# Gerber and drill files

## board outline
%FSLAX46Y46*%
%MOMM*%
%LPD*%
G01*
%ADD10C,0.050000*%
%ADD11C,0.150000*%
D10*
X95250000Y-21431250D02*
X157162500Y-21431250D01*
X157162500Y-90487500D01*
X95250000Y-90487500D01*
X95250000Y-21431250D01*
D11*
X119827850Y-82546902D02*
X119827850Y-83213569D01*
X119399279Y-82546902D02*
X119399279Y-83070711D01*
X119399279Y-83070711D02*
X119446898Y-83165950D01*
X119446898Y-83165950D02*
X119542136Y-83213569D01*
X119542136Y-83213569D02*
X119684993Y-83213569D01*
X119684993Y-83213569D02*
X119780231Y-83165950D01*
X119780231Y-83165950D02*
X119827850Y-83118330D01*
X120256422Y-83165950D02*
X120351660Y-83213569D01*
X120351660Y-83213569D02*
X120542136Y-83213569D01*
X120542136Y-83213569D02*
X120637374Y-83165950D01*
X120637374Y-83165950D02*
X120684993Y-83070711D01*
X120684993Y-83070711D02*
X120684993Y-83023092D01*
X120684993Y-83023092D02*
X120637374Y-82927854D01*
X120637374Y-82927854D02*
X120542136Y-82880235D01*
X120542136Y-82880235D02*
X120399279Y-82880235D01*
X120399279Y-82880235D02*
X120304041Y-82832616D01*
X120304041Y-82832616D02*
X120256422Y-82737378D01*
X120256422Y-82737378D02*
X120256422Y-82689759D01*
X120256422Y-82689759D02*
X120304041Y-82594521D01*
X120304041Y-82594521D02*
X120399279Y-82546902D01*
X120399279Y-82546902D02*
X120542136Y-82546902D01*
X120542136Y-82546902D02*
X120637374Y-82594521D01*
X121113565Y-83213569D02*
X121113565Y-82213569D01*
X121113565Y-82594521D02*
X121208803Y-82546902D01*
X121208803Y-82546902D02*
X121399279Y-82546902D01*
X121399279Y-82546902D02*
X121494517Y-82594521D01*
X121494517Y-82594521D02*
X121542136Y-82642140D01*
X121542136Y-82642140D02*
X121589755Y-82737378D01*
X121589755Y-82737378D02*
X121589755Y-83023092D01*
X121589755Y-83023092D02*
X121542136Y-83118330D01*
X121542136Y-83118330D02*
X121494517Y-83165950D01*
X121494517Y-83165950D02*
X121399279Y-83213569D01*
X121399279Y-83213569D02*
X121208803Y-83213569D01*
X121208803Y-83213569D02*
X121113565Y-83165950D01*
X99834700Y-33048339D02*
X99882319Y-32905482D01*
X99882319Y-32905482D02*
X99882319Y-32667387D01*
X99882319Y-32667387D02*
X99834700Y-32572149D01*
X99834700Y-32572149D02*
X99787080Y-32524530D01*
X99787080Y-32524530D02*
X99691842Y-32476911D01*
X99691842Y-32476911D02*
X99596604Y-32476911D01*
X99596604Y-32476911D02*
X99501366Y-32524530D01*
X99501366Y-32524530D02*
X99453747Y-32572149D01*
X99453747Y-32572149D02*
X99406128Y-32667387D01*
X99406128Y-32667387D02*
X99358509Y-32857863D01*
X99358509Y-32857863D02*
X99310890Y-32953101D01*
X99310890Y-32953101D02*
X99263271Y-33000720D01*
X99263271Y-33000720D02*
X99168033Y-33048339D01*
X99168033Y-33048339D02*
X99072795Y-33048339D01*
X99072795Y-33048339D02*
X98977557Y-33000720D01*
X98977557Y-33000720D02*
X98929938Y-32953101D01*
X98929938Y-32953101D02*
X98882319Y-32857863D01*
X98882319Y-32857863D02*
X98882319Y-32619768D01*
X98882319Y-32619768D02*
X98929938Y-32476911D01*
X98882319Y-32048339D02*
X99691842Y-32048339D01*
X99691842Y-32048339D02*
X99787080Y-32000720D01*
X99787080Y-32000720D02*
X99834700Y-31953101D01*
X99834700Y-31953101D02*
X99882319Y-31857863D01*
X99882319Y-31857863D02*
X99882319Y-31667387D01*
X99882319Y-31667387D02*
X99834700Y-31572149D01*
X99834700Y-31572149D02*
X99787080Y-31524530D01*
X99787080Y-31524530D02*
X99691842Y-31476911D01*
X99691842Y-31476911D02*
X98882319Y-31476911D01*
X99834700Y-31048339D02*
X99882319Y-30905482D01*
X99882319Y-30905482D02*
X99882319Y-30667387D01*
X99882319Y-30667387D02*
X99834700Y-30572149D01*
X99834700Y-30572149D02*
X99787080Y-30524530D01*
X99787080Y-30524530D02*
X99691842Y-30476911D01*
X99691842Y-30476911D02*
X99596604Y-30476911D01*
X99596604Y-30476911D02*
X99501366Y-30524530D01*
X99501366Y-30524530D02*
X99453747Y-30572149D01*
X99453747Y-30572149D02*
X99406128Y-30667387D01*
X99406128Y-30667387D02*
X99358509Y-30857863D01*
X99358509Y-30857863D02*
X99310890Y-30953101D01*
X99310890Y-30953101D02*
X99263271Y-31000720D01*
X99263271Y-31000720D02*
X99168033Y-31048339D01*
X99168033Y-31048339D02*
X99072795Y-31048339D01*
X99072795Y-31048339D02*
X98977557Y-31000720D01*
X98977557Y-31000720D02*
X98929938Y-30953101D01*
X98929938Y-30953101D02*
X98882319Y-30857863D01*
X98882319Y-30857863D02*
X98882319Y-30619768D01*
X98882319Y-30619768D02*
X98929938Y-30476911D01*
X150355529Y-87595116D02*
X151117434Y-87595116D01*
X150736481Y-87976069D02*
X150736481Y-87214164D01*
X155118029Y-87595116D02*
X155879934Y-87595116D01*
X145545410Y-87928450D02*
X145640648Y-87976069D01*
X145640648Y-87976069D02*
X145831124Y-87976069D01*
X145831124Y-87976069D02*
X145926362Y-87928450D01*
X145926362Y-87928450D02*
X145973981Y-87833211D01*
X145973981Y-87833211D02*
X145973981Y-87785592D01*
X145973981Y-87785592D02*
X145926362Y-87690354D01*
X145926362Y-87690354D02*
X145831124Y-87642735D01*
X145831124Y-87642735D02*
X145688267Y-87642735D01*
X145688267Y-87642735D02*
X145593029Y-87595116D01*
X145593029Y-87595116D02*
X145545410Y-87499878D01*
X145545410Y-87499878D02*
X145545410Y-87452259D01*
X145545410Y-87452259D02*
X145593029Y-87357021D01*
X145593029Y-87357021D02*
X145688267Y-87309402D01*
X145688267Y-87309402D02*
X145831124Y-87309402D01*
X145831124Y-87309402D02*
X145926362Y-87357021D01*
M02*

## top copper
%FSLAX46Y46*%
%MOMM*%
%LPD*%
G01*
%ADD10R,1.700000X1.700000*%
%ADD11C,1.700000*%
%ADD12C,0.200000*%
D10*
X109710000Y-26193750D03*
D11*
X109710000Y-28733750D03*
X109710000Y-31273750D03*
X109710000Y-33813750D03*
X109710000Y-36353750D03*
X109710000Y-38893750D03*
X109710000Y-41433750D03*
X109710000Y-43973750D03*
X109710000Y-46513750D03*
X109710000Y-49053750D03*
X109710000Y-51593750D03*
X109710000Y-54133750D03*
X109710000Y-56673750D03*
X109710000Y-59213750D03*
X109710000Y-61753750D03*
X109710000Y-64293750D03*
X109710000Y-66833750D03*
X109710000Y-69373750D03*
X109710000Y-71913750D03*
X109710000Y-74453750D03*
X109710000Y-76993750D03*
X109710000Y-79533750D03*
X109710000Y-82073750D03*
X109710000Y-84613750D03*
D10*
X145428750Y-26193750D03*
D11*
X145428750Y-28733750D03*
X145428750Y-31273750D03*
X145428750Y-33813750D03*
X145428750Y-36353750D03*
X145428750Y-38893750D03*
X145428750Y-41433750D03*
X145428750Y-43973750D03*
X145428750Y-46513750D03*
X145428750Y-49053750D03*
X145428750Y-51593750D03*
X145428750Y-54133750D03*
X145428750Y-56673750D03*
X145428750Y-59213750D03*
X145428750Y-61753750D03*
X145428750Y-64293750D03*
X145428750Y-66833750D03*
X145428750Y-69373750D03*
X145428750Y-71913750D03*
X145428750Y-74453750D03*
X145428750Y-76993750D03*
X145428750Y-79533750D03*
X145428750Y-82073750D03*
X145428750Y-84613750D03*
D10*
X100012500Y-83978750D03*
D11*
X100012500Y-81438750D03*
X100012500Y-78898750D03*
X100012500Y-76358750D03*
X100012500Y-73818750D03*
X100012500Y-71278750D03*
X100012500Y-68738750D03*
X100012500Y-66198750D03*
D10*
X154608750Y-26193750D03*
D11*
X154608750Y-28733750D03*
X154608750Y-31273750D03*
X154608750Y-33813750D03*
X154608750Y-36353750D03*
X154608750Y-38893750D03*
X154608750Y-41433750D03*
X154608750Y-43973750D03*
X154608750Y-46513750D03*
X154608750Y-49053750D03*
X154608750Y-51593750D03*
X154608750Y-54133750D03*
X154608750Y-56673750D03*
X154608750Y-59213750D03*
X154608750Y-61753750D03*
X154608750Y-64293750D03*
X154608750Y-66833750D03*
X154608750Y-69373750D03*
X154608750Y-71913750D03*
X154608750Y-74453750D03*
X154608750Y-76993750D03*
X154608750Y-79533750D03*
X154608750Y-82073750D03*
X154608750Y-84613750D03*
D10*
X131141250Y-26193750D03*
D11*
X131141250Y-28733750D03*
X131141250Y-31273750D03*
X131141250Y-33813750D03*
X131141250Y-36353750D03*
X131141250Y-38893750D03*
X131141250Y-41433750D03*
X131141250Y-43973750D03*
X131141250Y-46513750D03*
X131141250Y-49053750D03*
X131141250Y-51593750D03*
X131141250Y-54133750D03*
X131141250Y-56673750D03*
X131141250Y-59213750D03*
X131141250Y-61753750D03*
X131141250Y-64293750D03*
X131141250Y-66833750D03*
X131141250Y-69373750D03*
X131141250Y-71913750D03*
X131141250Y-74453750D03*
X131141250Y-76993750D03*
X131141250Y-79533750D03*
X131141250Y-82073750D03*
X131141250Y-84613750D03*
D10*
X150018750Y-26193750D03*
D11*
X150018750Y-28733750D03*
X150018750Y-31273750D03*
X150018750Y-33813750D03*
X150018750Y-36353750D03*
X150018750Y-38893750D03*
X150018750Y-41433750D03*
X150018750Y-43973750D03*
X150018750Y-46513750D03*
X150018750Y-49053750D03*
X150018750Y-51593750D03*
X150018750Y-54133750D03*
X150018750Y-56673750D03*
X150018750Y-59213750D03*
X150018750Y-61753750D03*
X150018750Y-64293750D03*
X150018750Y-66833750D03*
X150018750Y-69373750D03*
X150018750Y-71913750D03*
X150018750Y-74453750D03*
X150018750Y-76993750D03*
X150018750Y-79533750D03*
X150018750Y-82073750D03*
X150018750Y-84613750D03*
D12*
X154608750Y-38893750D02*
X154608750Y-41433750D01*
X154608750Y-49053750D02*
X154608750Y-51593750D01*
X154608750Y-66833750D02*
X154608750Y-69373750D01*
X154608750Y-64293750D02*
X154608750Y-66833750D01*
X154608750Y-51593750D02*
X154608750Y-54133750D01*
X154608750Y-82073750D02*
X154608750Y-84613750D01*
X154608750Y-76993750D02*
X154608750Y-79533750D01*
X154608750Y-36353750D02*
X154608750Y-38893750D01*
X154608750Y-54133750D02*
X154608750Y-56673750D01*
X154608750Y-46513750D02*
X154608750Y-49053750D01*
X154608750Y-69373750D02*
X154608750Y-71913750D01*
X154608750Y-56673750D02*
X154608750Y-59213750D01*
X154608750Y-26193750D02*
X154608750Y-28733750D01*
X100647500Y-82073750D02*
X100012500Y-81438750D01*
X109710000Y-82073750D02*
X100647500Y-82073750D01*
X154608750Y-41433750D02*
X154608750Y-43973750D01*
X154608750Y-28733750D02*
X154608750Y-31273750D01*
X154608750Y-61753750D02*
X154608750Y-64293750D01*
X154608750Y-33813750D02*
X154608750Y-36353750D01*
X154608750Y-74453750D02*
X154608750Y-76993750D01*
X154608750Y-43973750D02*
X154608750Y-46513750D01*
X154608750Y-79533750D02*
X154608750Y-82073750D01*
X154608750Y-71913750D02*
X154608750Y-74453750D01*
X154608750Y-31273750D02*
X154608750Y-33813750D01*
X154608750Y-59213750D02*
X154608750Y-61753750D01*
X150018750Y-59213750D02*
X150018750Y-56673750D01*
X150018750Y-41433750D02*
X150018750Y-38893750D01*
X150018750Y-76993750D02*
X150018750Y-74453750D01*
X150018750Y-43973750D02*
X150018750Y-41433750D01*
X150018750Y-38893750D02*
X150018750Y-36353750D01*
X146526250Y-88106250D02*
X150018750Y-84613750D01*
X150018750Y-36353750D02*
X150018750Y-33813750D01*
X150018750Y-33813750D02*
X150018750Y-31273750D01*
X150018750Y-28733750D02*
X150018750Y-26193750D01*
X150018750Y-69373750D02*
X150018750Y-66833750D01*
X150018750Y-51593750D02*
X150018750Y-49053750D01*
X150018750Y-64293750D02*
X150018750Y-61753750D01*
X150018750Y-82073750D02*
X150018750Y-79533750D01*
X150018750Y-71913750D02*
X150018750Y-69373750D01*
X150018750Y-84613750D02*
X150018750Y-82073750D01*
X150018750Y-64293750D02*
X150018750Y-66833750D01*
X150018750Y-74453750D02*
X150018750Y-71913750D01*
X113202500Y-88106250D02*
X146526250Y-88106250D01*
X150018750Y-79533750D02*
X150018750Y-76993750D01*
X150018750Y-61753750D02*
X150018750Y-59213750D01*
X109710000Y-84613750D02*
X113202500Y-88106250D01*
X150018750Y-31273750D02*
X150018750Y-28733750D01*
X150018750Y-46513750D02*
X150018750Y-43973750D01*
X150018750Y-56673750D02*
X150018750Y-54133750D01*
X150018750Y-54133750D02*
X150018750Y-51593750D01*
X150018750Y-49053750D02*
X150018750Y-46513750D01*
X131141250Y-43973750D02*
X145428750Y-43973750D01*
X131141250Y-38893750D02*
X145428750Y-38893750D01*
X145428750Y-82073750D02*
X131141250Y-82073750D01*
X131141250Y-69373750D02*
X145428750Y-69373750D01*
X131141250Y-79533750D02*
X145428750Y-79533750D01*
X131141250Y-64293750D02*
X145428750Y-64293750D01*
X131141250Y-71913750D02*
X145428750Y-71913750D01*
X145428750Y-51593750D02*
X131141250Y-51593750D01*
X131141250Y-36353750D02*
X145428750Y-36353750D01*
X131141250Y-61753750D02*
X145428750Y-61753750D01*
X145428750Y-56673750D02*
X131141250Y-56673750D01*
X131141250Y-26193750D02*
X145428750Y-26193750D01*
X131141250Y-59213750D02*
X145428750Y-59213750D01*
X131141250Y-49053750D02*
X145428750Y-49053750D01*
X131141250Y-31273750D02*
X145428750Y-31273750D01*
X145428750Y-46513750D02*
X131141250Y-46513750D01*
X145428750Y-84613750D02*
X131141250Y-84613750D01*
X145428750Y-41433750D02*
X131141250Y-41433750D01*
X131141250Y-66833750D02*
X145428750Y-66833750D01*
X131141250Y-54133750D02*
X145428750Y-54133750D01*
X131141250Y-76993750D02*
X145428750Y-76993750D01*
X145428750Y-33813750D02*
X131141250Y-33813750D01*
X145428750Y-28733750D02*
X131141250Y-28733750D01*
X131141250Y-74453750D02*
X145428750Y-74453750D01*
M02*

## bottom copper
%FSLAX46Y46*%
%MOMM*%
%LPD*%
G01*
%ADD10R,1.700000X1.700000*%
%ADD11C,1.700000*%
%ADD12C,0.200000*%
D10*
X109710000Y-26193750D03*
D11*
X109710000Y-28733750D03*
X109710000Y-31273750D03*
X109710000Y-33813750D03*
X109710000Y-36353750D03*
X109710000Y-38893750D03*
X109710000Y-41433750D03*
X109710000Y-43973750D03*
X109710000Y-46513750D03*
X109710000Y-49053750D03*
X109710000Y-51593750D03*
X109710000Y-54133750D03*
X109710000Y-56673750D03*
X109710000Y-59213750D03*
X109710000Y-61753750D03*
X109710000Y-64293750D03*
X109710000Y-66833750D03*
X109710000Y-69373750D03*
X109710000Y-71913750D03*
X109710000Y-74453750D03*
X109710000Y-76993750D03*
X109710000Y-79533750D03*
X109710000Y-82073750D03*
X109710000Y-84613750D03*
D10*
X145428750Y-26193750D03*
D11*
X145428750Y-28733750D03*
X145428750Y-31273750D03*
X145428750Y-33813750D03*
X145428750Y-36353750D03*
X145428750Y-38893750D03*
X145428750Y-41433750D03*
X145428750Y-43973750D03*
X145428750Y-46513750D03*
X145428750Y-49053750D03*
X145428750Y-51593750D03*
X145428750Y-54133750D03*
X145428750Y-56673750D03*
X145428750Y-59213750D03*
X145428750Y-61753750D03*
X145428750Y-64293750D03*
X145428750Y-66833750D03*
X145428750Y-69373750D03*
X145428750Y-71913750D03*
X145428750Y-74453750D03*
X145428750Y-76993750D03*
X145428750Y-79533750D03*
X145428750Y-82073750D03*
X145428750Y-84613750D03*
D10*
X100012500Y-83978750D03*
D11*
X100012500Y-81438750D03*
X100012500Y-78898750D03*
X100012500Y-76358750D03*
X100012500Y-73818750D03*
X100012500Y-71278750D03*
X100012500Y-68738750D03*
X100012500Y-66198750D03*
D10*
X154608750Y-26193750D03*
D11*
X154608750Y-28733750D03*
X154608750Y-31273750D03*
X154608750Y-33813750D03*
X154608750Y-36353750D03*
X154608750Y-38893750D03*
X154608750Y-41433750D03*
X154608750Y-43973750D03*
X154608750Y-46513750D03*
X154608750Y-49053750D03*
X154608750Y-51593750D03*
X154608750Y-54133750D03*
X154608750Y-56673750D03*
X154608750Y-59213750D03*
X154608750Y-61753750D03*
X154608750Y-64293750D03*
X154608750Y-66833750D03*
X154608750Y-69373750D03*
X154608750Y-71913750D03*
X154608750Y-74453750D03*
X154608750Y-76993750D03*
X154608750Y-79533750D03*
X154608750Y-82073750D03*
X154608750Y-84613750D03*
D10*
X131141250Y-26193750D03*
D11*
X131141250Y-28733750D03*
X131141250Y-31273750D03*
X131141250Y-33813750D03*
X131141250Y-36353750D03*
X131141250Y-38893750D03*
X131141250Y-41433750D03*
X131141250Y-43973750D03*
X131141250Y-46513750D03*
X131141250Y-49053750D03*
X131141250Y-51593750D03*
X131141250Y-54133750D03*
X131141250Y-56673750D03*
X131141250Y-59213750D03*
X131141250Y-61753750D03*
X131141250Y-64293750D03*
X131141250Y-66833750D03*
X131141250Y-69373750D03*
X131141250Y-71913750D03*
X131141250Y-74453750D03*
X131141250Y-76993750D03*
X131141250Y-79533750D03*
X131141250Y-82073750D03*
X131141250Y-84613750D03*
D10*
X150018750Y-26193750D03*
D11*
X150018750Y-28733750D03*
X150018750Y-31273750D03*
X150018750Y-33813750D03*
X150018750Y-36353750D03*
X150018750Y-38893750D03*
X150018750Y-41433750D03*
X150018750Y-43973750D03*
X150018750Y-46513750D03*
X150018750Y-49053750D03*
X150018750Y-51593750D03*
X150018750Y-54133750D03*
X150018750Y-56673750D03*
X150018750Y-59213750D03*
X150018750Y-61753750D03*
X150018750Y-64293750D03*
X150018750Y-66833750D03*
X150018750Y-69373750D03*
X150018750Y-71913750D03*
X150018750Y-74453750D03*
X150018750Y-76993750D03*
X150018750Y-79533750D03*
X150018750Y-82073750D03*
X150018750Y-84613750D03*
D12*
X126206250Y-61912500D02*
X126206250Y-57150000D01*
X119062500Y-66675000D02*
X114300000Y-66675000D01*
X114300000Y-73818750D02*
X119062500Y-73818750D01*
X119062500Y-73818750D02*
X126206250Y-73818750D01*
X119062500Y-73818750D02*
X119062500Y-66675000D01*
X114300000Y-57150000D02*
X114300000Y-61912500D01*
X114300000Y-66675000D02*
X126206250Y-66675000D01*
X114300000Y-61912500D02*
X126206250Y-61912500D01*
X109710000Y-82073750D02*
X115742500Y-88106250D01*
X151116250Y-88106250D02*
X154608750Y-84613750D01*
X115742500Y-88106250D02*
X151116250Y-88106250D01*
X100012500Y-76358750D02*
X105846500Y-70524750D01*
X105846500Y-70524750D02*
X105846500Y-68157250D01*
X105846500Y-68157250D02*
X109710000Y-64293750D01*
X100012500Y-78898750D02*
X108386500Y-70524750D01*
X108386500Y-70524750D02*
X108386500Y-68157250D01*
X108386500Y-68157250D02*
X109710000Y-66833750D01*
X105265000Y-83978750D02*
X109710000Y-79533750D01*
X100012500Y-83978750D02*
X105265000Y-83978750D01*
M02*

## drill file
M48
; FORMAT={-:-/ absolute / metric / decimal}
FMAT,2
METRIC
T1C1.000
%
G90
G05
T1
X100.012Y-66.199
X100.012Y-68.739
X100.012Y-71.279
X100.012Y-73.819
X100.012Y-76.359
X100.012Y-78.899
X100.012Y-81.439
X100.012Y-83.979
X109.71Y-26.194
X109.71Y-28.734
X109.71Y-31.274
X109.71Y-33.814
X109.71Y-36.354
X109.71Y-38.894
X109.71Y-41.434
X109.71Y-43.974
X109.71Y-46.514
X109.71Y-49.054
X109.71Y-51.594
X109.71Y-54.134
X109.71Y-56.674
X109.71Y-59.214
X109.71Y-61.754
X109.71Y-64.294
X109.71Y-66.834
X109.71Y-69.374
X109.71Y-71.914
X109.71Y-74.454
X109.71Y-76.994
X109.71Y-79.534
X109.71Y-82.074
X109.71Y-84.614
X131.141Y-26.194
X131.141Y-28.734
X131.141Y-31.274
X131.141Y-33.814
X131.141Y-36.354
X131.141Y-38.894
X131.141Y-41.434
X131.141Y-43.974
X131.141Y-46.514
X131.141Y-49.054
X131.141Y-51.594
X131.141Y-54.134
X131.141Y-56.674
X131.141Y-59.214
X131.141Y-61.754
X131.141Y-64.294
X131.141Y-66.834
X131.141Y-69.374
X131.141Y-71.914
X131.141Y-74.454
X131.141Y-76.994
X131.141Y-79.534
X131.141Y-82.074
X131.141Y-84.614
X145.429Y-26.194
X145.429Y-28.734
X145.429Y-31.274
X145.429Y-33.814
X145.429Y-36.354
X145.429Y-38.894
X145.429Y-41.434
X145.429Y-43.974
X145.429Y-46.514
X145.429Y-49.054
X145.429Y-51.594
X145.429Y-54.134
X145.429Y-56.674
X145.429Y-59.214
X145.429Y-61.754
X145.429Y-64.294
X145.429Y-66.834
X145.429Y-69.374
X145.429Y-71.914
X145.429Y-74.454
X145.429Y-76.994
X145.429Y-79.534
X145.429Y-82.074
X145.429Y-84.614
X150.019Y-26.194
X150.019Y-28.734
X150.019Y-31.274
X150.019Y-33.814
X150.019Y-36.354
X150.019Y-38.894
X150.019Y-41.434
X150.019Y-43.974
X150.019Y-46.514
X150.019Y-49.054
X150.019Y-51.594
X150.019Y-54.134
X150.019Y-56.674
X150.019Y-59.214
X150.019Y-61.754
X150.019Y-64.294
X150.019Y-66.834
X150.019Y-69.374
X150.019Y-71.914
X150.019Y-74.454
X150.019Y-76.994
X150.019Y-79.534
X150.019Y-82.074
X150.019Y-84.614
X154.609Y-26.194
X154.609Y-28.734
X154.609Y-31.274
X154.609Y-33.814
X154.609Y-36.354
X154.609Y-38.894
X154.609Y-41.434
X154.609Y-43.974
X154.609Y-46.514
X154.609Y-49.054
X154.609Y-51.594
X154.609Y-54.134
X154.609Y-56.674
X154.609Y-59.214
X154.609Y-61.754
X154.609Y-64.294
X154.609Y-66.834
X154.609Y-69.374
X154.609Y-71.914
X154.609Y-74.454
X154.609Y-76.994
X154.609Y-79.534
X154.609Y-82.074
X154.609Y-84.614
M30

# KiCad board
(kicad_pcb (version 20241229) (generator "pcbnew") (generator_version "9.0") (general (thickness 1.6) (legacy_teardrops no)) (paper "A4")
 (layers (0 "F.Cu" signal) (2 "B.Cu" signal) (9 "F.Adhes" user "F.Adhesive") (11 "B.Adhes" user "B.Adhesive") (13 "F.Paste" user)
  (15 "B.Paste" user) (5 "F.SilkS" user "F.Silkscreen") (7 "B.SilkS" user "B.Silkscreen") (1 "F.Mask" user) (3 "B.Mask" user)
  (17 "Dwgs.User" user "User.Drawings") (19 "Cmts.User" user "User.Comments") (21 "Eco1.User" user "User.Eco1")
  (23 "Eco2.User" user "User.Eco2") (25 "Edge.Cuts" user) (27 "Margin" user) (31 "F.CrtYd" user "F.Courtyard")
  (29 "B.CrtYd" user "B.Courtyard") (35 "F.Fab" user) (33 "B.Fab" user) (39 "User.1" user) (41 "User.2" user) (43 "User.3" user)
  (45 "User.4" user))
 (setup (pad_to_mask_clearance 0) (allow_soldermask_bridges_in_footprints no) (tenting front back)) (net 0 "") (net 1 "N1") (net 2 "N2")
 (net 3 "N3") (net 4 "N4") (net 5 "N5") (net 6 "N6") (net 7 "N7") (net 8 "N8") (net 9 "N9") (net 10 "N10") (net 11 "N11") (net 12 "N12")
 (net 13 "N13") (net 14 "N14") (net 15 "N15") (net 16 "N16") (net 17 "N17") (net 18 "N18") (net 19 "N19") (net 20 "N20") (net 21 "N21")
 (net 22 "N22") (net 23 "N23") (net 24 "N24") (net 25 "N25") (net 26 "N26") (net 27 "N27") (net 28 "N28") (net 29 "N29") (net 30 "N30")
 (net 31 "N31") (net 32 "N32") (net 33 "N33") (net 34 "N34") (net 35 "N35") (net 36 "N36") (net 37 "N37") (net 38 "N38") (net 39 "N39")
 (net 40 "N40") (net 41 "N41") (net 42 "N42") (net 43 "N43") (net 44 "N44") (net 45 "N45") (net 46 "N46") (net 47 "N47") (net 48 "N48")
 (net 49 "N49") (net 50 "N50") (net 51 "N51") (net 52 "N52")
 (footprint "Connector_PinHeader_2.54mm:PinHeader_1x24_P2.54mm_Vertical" (layer "F.Cu") (at 109.71 26.19375)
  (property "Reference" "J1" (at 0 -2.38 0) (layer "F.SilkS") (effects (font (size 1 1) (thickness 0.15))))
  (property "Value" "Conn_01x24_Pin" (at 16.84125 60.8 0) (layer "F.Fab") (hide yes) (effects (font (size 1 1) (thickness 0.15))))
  (pad "1" thru_hole rect (at 0 0) (size 1.7 1.7) (drill 1) (layers "*.Cu" "*.Mask") (remove_unused_layers no) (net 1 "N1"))
  (pad "2" thru_hole circle (at 0 2.54) (size 1.7 1.7) (drill 1) (layers "*.Cu" "*.Mask") (remove_unused_layers no) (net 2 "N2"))
  (pad "3" thru_hole circle (at 0 5.08) (size 1.7 1.7) (drill 1) (layers "*.Cu" "*.Mask") (remove_unused_layers no) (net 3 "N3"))
  (pad "4" thru_hole circle (at 0 7.62) (size 1.7 1.7) (drill 1) (layers "*.Cu" "*.Mask") (remove_unused_layers no) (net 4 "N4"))
  (pad "5" thru_hole circle (at 0 10.16) (size 1.7 1.7) (drill 1) (layers "*.Cu" "*.Mask") (remove_unused_layers no) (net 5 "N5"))
  (pad "6" thru_hole circle (at 0 12.7) (size 1.7 1.7) (drill 1) (layers "*.Cu" "*.Mask") (remove_unused_layers no) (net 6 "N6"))
  (pad "7" thru_hole circle (at 0 15.24) (size 1.7 1.7) (drill 1) (layers "*.Cu" "*.Mask") (remove_unused_layers no) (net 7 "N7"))
  (pad "8" thru_hole circle (at 0 17.78) (size 1.7 1.7) (drill 1) (layers "*.Cu" "*.Mask") (remove_unused_layers no) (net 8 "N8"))
  (pad "9" thru_hole circle (at 0 20.32) (size 1.7 1.7) (drill 1) (layers "*.Cu" "*.Mask") (remove_unused_layers no) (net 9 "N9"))
  (pad "10" thru_hole circle (at 0 22.86) (size 1.7 1.7) (drill 1) (layers "*.Cu" "*.Mask") (remove_unused_layers no) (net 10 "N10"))
  (pad "11" thru_hole circle (at 0 25.4) (size 1.7 1.7) (drill 1) (layers "*.Cu" "*.Mask") (remove_unused_layers no) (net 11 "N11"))
  (pad "12" thru_hole circle (at 0 27.94) (size 1.7 1.7) (drill 1) (layers "*.Cu" "*.Mask") (remove_unused_layers no) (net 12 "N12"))
  (pad "13" thru_hole circle (at 0 30.48) (size 1.7 1.7) (drill 1) (layers "*.Cu" "*.Mask") (remove_unused_layers no) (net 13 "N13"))
  (pad "14" thru_hole circle (at 0 33.02) (size 1.7 1.7) (drill 1) (layers "*.Cu" "*.Mask") (remove_unused_layers no) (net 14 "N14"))
  (pad "15" thru_hole circle (at 0 35.56) (size 1.7 1.7) (drill 1) (layers "*.Cu" "*.Mask") (remove_unused_layers no) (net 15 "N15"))
  (pad "16" thru_hole circle (at 0 38.1) (size 1.7 1.7) (drill 1) (layers "*.Cu" "*.Mask") (remove_unused_layers no) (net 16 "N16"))
  (pad "17" thru_hole circle (at 0 40.64) (size 1.7 1.7) (drill 1) (layers "*.Cu" "*.Mask") (remove_unused_layers no) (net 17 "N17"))
  (pad "18" thru_hole circle (at 0 43.18) (size 1.7 1.7) (drill 1) (layers "*.Cu" "*.Mask") (remove_unused_layers no) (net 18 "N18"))
  (pad "19" thru_hole circle (at 0 45.72) (size 1.7 1.7) (drill 1) (layers "*.Cu" "*.Mask") (remove_unused_layers no) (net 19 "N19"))
  (pad "20" thru_hole circle (at 0 48.26) (size 1.7 1.7) (drill 1) (layers "*.Cu" "*.Mask") (remove_unused_layers no) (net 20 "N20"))
  (pad "21" thru_hole circle (at 0 50.8) (size 1.7 1.7) (drill 1) (layers "*.Cu" "*.Mask") (remove_unused_layers no) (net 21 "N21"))
  (pad "22" thru_hole circle (at 0 53.34) (size 1.7 1.7) (drill 1) (layers "*.Cu" "*.Mask") (remove_unused_layers no) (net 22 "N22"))
  (pad "23" thru_hole circle (at 0 55.88) (size 1.7 1.7) (drill 1) (layers "*.Cu" "*.Mask") (remove_unused_layers no) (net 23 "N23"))
  (pad "24" thru_hole circle (at 0 58.42) (size 1.7 1.7) (drill 1) (layers "*.Cu" "*.Mask") (remove_unused_layers no) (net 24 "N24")))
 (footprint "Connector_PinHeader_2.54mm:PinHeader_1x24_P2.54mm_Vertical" (layer "F.Cu") (at 145.42875 26.19375)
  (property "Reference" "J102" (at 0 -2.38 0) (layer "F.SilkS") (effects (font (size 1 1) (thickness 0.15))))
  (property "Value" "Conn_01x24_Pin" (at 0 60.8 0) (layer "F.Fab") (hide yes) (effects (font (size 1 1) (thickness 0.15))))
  (pad "1" thru_hole rect (at 0 0) (size 1.7 1.7) (drill 1) (layers "*.Cu" "*.Mask") (remove_unused_layers no) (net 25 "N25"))
  (pad "2" thru_hole circle (at 0 2.54) (size 1.7 1.7) (drill 1) (layers "*.Cu" "*.Mask") (remove_unused_layers no) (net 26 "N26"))
  (pad "3" thru_hole circle (at 0 5.08) (size 1.7 1.7) (drill 1) (layers "*.Cu" "*.Mask") (remove_unused_layers no) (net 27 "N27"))
  (pad "4" thru_hole circle (at 0 7.62) (size 1.7 1.7) (drill 1) (layers "*.Cu" "*.Mask") (remove_unused_layers no) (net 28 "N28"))
  (pad "5" thru_hole circle (at 0 10.16) (size 1.7 1.7) (drill 1) (layers "*.Cu" "*.Mask") (remove_unused_layers no) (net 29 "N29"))
  (pad "6" thru_hole circle (at 0 12.7) (size 1.7 1.7) (drill 1) (layers "*.Cu" "*.Mask") (remove_unused_layers no) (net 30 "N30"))
  (pad "7" thru_hole circle (at 0 15.24) (size 1.7 1.7) (drill 1) (layers "*.Cu" "*.Mask") (remove_unused_layers no) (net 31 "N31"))
  (pad "8" thru_hole circle (at 0 17.78) (size 1.7 1.7) (drill 1) (layers "*.Cu" "*.Mask") (remove_unused_layers no) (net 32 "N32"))
  (pad "9" thru_hole circle (at 0 20.32) (size 1.7 1.7) (drill 1) (layers "*.Cu" "*.Mask") (remove_unused_layers no) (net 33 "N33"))
  (pad "10" thru_hole circle (at 0 22.86) (size 1.7 1.7) (drill 1) (layers "*.Cu" "*.Mask") (remove_unused_layers no) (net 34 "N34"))
  (pad "11" thru_hole circle (at 0 25.4) (size 1.7 1.7) (drill 1) (layers "*.Cu" "*.Mask") (remove_unused_layers no) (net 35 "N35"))
  (pad "12" thru_hole circle (at 0 27.94) (size 1.7 1.7) (drill 1) (layers "*.Cu" "*.Mask") (remove_unused_layers no) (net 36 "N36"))
  (pad "13" thru_hole circle (at 0 30.48) (size 1.7 1.7) (drill 1) (layers "*.Cu" "*.Mask") (remove_unused_layers no) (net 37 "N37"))
  (pad "14" thru_hole circle (at 0 33.02) (size 1.7 1.7) (drill 1) (layers "*.Cu" "*.Mask") (remove_unused_layers no) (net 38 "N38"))
  (pad "15" thru_hole circle (at 0 35.56) (size 1.7 1.7) (drill 1) (layers "*.Cu" "*.Mask") (remove_unused_layers no) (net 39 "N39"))
  (pad "16" thru_hole circle (at 0 38.1) (size 1.7 1.7) (drill 1) (layers "*.Cu" "*.Mask") (remove_unused_layers no) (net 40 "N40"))
  (pad "17" thru_hole circle (at 0 40.64) (size 1.7 1.7) (drill 1) (layers "*.Cu" "*.Mask") (remove_unused_layers no) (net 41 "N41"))
  (pad "18" thru_hole circle (at 0 43.18) (size 1.7 1.7) (drill 1) (layers "*.Cu" "*.Mask") (remove_unused_layers no) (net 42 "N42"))
  (pad "19" thru_hole circle (at 0 45.72) (size 1.7 1.7) (drill 1) (layers "*.Cu" "*.Mask") (remove_unused_layers no) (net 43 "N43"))
  (pad "20" thru_hole circle (at 0 48.26) (size 1.7 1.7) (drill 1) (layers "*.Cu" "*.Mask") (remove_unused_layers no) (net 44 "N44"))
  (pad "21" thru_hole circle (at 0 50.8) (size 1.7 1.7) (drill 1) (layers "*.Cu" "*.Mask") (remove_unused_layers no) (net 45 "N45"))
  (pad "22" thru_hole circle (at 0 53.34) (size 1.7 1.7) (drill 1) (layers "*.Cu" "*.Mask") (remove_unused_layers no) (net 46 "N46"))
  (pad "23" thru_hole circle (at 0 55.88) (size 1.7 1.7) (drill 1) (layers "*.Cu" "*.Mask") (remove_unused_layers no) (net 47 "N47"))
  (pad "24" thru_hole circle (at 0 58.42) (size 1.7 1.7) (drill 1) (layers "*.Cu" "*.Mask") (remove_unused_layers no) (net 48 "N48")))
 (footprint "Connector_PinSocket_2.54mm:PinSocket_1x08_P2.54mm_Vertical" (layer "F.Cu") (at 100.0125 83.97875 180)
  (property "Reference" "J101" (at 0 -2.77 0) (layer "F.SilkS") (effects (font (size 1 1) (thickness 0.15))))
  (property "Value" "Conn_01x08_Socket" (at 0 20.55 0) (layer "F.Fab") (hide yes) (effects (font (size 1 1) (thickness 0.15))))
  (pad "1" thru_hole rect (at 0 0 180) (size 1.7 1.7) (drill 1) (layers "*.Cu" "*.Mask") (remove_unused_layers no) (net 22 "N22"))
  (pad "2" thru_hole circle (at 0 2.54 180) (size 1.7 1.7) (drill 1) (layers "*.Cu" "*.Mask") (remove_unused_layers no) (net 23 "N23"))
  (pad "3" thru_hole circle (at 0 5.08 180) (size 1.7 1.7) (drill 1) (layers "*.Cu" "*.Mask") (remove_unused_layers no) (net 17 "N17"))
  (pad "4" thru_hole circle (at 0 7.62 180) (size 1.7 1.7) (drill 1) (layers "*.Cu" "*.Mask") (remove_unused_layers no) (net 16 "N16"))
  (pad "5" thru_hole circle (at 0 10.16 180) (size 1.7 1.7) (drill 1) (layers "*.Cu" "*.Mask") (remove_unused_layers no) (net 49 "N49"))
  (pad "6" thru_hole circle (at 0 12.7 180) (size 1.7 1.7) (drill 1) (layers "*.Cu" "*.Mask") (remove_unused_layers no) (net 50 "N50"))
  (pad "7" thru_hole circle (at 0 15.24 180) (size 1.7 1.7) (drill 1) (layers "*.Cu" "*.Mask") (remove_unused_layers no) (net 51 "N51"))
  (pad "8" thru_hole circle (at 0 17.78 180) (size 1.7 1.7) (drill 1) (layers "*.Cu" "*.Mask") (remove_unused_layers no) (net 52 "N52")))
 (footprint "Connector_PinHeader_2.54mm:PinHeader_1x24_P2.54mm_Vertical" (layer "F.Cu") (at 154.60875 26.19375)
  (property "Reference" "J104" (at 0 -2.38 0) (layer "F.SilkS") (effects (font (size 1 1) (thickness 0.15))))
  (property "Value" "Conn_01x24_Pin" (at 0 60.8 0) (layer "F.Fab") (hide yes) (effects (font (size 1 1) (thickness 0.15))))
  (pad "1" thru_hole rect (at 0 0) (size 1.7 1.7) (drill 1) (layers "*.Cu" "*.Mask") (remove_unused_layers no) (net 23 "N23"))
  (pad "2" thru_hole circle (at 0 2.54) (size 1.7 1.7) (drill 1) (layers "*.Cu" "*.Mask") (remove_unused_layers no) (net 23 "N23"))
  (pad "3" thru_hole circle (at 0 5.08) (size 1.7 1.7) (drill 1) (layers "*.Cu" "*.Mask") (remove_unused_layers no) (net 23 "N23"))
  (pad "4" thru_hole circle (at 0 7.62) (size 1.7 1.7) (drill 1) (layers "*.Cu" "*.Mask") (remove_unused_layers no) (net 23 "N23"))
  (pad "5" thru_hole circle (at 0 10.16) (size 1.7 1.7) (drill 1) (layers "*.Cu" "*.Mask") (remove_unused_layers no) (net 23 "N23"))
  (pad "6" thru_hole circle (at 0 12.7) (size 1.7 1.7) (drill 1) (layers "*.Cu" "*.Mask") (remove_unused_layers no) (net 23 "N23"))
  (pad "7" thru_hole circle (at 0 15.24) (size 1.7 1.7) (drill 1) (layers "*.Cu" "*.Mask") (remove_unused_layers no) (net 23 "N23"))
  (pad "8" thru_hole circle (at 0 17.78) (size 1.7 1.7) (drill 1) (layers "*.Cu" "*.Mask") (remove_unused_layers no) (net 23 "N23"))
  (pad "9" thru_hole circle (at 0 20.32) (size 1.7 1.7) (drill 1) (layers "*.Cu" "*.Mask") (remove_unused_layers no) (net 23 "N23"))
  (pad "10" thru_hole circle (at 0 22.86) (size 1.7 1.7) (drill 1) (layers "*.Cu" "*.Mask") (remove_unused_layers no) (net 23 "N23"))
  (pad "11" thru_hole circle (at 0 25.4) (size 1.7 1.7) (drill 1) (layers "*.Cu" "*.Mask") (remove_unused_layers no) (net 23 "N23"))
  (pad "12" thru_hole circle (at 0 27.94) (size 1.7 1.7) (drill 1) (layers "*.Cu" "*.Mask") (remove_unused_layers no) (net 23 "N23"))
  (pad "13" thru_hole circle (at 0 30.48) (size 1.7 1.7) (drill 1) (layers "*.Cu" "*.Mask") (remove_unused_layers no) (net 23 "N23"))
  (pad "14" thru_hole circle (at 0 33.02) (size 1.7 1.7) (drill 1) (layers "*.Cu" "*.Mask") (remove_unused_layers no) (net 23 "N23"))
  (pad "15" thru_hole circle (at 0 35.56) (size 1.7 1.7) (drill 1) (layers "*.Cu" "*.Mask") (remove_unused_layers no) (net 23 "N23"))
  (pad "16" thru_hole circle (at 0 38.1) (size 1.7 1.7) (drill 1) (layers "*.Cu" "*.Mask") (remove_unused_layers no) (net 23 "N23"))
  (pad "17" thru_hole circle (at 0 40.64) (size 1.7 1.7) (drill 1) (layers "*.Cu" "*.Mask") (remove_unused_layers no) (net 23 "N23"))
  (pad "18" thru_hole circle (at 0 43.18) (size 1.7 1.7) (drill 1) (layers "*.Cu" "*.Mask") (remove_unused_layers no) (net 23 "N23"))
  (pad "19" thru_hole circle (at 0 45.72) (size 1.7 1.7) (drill 1) (layers "*.Cu" "*.Mask") (remove_unused_layers no) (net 23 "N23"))
  (pad "20" thru_hole circle (at 0 48.26) (size 1.7 1.7) (drill 1) (layers "*.Cu" "*.Mask") (remove_unused_layers no) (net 23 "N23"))
  (pad "21" thru_hole circle (at 0 50.8) (size 1.7 1.7) (drill 1) (layers "*.Cu" "*.Mask") (remove_unused_layers no) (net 23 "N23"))
  (pad "22" thru_hole circle (at 0 53.34) (size 1.7 1.7) (drill 1) (layers "*.Cu" "*.Mask") (remove_unused_layers no) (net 23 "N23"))
  (pad "23" thru_hole circle (at 0 55.88) (size 1.7 1.7) (drill 1) (layers "*.Cu" "*.Mask") (remove_unused_layers no) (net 23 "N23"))
  (pad "24" thru_hole circle (at 0 58.42) (size 1.7 1.7) (drill 1) (layers "*.Cu" "*.Mask") (remove_unused_layers no) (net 23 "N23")))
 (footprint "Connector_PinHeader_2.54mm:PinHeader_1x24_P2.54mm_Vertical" (layer "F.Cu") (at 131.14125 26.19375)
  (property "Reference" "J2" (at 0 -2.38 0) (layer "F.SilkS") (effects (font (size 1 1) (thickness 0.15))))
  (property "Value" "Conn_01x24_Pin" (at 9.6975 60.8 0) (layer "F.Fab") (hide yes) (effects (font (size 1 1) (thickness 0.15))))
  (pad "1" thru_hole rect (at 0 0) (size 1.7 1.7) (drill 1) (layers "*.Cu" "*.Mask") (remove_unused_layers no) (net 25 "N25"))
  (pad "2" thru_hole circle (at 0 2.54) (size 1.7 1.7) (drill 1) (layers "*.Cu" "*.Mask") (remove_unused_layers no) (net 26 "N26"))
  (pad "3" thru_hole circle (at 0 5.08) (size 1.7 1.7) (drill 1) (layers "*.Cu" "*.Mask") (remove_unused_layers no) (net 27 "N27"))
  (pad "4" thru_hole circle (at 0 7.62) (size 1.7 1.7) (drill 1) (layers "*.Cu" "*.Mask") (remove_unused_layers no) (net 28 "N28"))
  (pad "5" thru_hole circle (at 0 10.16) (size 1.7 1.7) (drill 1) (layers "*.Cu" "*.Mask") (remove_unused_layers no) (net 29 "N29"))
  (pad "6" thru_hole circle (at 0 12.7) (size 1.7 1.7) (drill 1) (layers "*.Cu" "*.Mask") (remove_unused_layers no) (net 30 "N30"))
  (pad "7" thru_hole circle (at 0 15.24) (size 1.7 1.7) (drill 1) (layers "*.Cu" "*.Mask") (remove_unused_layers no) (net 31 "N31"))
  (pad "8" thru_hole circle (at 0 17.78) (size 1.7 1.7) (drill 1) (layers "*.Cu" "*.Mask") (remove_unused_layers no) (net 32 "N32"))
  (pad "9" thru_hole circle (at 0 20.32) (size 1.7 1.7) (drill 1) (layers "*.Cu" "*.Mask") (remove_unused_layers no) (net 33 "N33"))
  (pad "10" thru_hole circle (at 0 22.86) (size 1.7 1.7) (drill 1) (layers "*.Cu" "*.Mask") (remove_unused_layers no) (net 34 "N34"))
  (pad "11" thru_hole circle (at 0 25.4) (size 1.7 1.7) (drill 1) (layers "*.Cu" "*.Mask") (remove_unused_layers no) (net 35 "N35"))
  (pad "12" thru_hole circle (at 0 27.94) (size 1.7 1.7) (drill 1) (layers "*.Cu" "*.Mask") (remove_unused_layers no) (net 36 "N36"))
  (pad "13" thru_hole circle (at 0 30.48) (size 1.7 1.7) (drill 1) (layers "*.Cu" "*.Mask") (remove_unused_layers no) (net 37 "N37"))
  (pad "14" thru_hole circle (at 0 33.02) (size 1.7 1.7) (drill 1) (layers "*.Cu" "*.Mask") (remove_unused_layers no) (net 38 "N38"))
  (pad "15" thru_hole circle (at 0 35.56) (size 1.7 1.7) (drill 1) (layers "*.Cu" "*.Mask") (remove_unused_layers no) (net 39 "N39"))
  (pad "16" thru_hole circle (at 0 38.1) (size 1.7 1.7) (drill 1) (layers "*.Cu" "*.Mask") (remove_unused_layers no) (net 40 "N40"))
  (pad "17" thru_hole circle (at 0 40.64) (size 1.7 1.7) (drill 1) (layers "*.Cu" "*.Mask") (remove_unused_layers no) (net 41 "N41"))
  (pad "18" thru_hole circle (at 0 43.18) (size 1.7 1.7) (drill 1) (layers "*.Cu" "*.Mask") (remove_unused_layers no) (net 42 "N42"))
  (pad "19" thru_hole circle (at 0 45.72) (size 1.7 1.7) (drill 1) (layers "*.Cu" "*.Mask") (remove_unused_layers no) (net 43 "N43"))
  (pad "20" thru_hole circle (at 0 48.26) (size 1.7 1.7) (drill 1) (layers "*.Cu" "*.Mask") (remove_unused_layers no) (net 44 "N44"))
  (pad "21" thru_hole circle (at 0 50.8) (size 1.7 1.7) (drill 1) (layers "*.Cu" "*.Mask") (remove_unused_layers no) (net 45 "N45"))
  (pad "22" thru_hole circle (at 0 53.34) (size 1.7 1.7) (drill 1) (layers "*.Cu" "*.Mask") (remove_unused_layers no) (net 46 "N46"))
  (pad "23" thru_hole circle (at 0 55.88) (size 1.7 1.7) (drill 1) (layers "*.Cu" "*.Mask") (remove_unused_layers no) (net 47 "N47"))
  (pad "24" thru_hole circle (at 0 58.42) (size 1.7 1.7) (drill 1) (layers "*.Cu" "*.Mask") (remove_unused_layers no) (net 48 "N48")))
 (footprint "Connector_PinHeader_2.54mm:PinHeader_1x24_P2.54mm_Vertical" (layer "F.Cu") (at 150.01875 26.19375)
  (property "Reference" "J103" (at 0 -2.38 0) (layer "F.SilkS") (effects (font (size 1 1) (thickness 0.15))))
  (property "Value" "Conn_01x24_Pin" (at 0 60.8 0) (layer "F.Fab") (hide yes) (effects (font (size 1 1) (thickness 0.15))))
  (pad "1" thru_hole rect (at 0 0) (size 1.7 1.7) (drill 1) (layers "*.Cu" "*.Mask") (remove_unused_layers no) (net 24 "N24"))
  (pad "2" thru_hole circle (at 0 2.54) (size 1.7 1.7) (drill 1) (layers "*.Cu" "*.Mask") (remove_unused_layers no) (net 24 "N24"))
  (pad "3" thru_hole circle (at 0 5.08) (size 1.7 1.7) (drill 1) (layers "*.Cu" "*.Mask") (remove_unused_layers no) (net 24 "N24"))
  (pad "4" thru_hole circle (at 0 7.62) (size 1.7 1.7) (drill 1) (layers "*.Cu" "*.Mask") (remove_unused_layers no) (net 24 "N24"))
  (pad "5" thru_hole circle (at 0 10.16) (size 1.7 1.7) (drill 1) (layers "*.Cu" "*.Mask") (remove_unused_layers no) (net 24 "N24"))
  (pad "6" thru_hole circle (at 0 12.7) (size 1.7 1.7) (drill 1) (layers "*.Cu" "*.Mask") (remove_unused_layers no) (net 24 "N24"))
  (pad "7" thru_hole circle (at 0 15.24) (size 1.7 1.7) (drill 1) (layers "*.Cu" "*.Mask") (remove_unused_layers no) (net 24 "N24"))
  (pad "8" thru_hole circle (at 0 17.78) (size 1.7 1.7) (drill 1) (layers "*.Cu" "*.Mask") (remove_unused_layers no) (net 24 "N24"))
  (pad "9" thru_hole circle (at 0 20.32) (size 1.7 1.7) (drill 1) (layers "*.Cu" "*.Mask") (remove_unused_layers no) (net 24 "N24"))
  (pad "10" thru_hole circle (at 0 22.86) (size 1.7 1.7) (drill 1) (layers "*.Cu" "*.Mask") (remove_unused_layers no) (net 24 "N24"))
  (pad "11" thru_hole circle (at 0 25.4) (size 1.7 1.7) (drill 1) (layers "*.Cu" "*.Mask") (remove_unused_layers no) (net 24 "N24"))
  (pad "12" thru_hole circle (at 0 27.94) (size 1.7 1.7) (drill 1) (layers "*.Cu" "*.Mask") (remove_unused_layers no) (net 24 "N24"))
  (pad "13" thru_hole circle (at 0 30.48) (size 1.7 1.7) (drill 1) (layers "*.Cu" "*.Mask") (remove_unused_layers no) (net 24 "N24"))
  (pad "14" thru_hole circle (at 0 33.02) (size 1.7 1.7) (drill 1) (layers "*.Cu" "*.Mask") (remove_unused_layers no) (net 24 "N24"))
  (pad "15" thru_hole circle (at 0 35.56) (size 1.7 1.7) (drill 1) (layers "*.Cu" "*.Mask") (remove_unused_layers no) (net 24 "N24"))
  (pad "16" thru_hole circle (at 0 38.1) (size 1.7 1.7) (drill 1) (layers "*.Cu" "*.Mask") (remove_unused_layers no) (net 24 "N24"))
  (pad "17" thru_hole circle (at 0 40.64) (size 1.7 1.7) (drill 1) (layers "*.Cu" "*.Mask") (remove_unused_layers no) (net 24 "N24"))
  (pad "18" thru_hole circle (at 0 43.18) (size 1.7 1.7) (drill 1) (layers "*.Cu" "*.Mask") (remove_unused_layers no) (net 24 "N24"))
  (pad "19" thru_hole circle (at 0 45.72) (size 1.7 1.7) (drill 1) (layers "*.Cu" "*.Mask") (remove_unused_layers no) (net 24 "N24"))
  (pad "20" thru_hole circle (at 0 48.26) (size 1.7 1.7) (drill 1) (layers "*.Cu" "*.Mask") (remove_unused_layers no) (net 24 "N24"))
  (pad "21" thru_hole circle (at 0 50.8) (size 1.7 1.7) (drill 1) (layers "*.Cu" "*.Mask") (remove_unused_layers no) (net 24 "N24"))
  (pad "22" thru_hole circle (at 0 53.34) (size 1.7 1.7) (drill 1) (layers "*.Cu" "*.Mask") (remove_unused_layers no) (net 24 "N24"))
  (pad "23" thru_hole circle (at 0 55.88) (size 1.7 1.7) (drill 1) (layers "*.Cu" "*.Mask") (remove_unused_layers no) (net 24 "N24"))
  (pad "24" thru_hole circle (at 0 58.42) (size 1.7 1.7) (drill 1) (layers "*.Cu" "*.Mask") (remove_unused_layers no) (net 24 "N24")))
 (gr_rect (start 95.25 21.43125) (end 157.1625 90.4875) (stroke (width 0.05) (type default)) (fill no) (layer "Edge.Cuts"))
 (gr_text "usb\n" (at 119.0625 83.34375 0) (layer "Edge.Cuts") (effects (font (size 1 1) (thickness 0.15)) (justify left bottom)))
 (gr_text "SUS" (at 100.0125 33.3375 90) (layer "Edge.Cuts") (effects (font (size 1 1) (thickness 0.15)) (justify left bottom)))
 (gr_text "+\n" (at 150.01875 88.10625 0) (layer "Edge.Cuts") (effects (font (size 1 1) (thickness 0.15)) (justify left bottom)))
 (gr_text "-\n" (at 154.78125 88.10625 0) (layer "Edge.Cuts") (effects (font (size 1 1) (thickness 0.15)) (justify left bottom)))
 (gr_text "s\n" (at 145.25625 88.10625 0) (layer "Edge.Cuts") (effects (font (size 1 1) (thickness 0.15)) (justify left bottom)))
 (segment (start 126.20625 61.9125) (end 126.20625 57.15) (width 0.2) (layer "B.Cu") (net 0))
 (segment (start 119.0625 66.675) (end 114.3 66.675) (width 0.2) (layer "B.Cu") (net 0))
 (segment (start 114.3 73.81875) (end 119.0625 73.81875) (width 0.2) (layer "B.Cu") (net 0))
 (segment (start 119.0625 73.81875) (end 126.20625 73.81875) (width 0.2) (layer "B.Cu") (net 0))
 (segment (start 119.0625 73.81875) (end 119.0625 66.675) (width 0.2) (layer "B.Cu") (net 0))
 (segment (start 114.3 57.15) (end 114.3 61.9125) (width 0.2) (layer "B.Cu") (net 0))
 (segment (start 114.3 66.675) (end 126.20625 66.675) (width 0.2) (layer "B.Cu") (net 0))
 (segment (start 114.3 61.9125) (end 126.20625 61.9125) (width 0.2) (layer "B.Cu") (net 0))
 (segment (start 154.60875 38.89375) (end 154.60875 41.43375) (width 0.2) (layer "F.Cu") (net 23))
 (segment (start 154.60875 49.05375) (end 154.60875 51.59375) (width 0.2) (layer "F.Cu") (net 23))
 (segment (start 154.60875 66.83375) (end 154.60875 69.37375) (width 0.2) (layer "F.Cu") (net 23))
 (segment (start 154.60875 64.29375) (end 154.60875 66.83375) (width 0.2) (layer "F.Cu") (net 23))
 (segment (start 154.60875 51.59375) (end 154.60875 54.13375) (width 0.2) (layer "F.Cu") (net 23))
 (segment (start 154.60875 82.07375) (end 154.60875 84.61375) (width 0.2) (layer "F.Cu") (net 23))
 (segment (start 154.60875 76.99375) (end 154.60875 79.53375) (width 0.2) (layer "F.Cu") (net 23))
 (segment (start 154.60875 36.35375) (end 154.60875 38.89375) (width 0.2) (layer "F.Cu") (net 23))
 (segment (start 154.60875 54.13375) (end 154.60875 56.67375) (width 0.2) (layer "F.Cu") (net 23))
 (segment (start 154.60875 46.51375) (end 154.60875 49.05375) (width 0.2) (layer "F.Cu") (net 23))
 (segment (start 154.60875 69.37375) (end 154.60875 71.91375) (width 0.2) (layer "F.Cu") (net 23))
 (segment (start 154.60875 56.67375) (end 154.60875 59.21375) (width 0.2) (layer "F.Cu") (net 23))
 (segment (start 154.60875 26.19375) (end 154.60875 28.73375) (width 0.2) (layer "F.Cu") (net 23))
 (segment (start 100.6475 82.07375) (end 100.0125 81.43875) (width 0.2) (layer "F.Cu") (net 23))
 (segment (start 109.71 82.07375) (end 100.6475 82.07375) (width 0.2) (layer "F.Cu") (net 23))
 (segment (start 154.60875 41.43375) (end 154.60875 43.97375) (width 0.2) (layer "F.Cu") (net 23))
 (segment (start 154.60875 28.73375) (end 154.60875 31.27375) (width 0.2) (layer "F.Cu") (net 23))
 (segment (start 154.60875 61.75375) (end 154.60875 64.29375) (width 0.2) (layer "F.Cu") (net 23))
 (segment (start 154.60875 33.81375) (end 154.60875 36.35375) (width 0.2) (layer "F.Cu") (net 23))
 (segment (start 154.60875 74.45375) (end 154.60875 76.99375) (width 0.2) (layer "F.Cu") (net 23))
 (segment (start 154.60875 43.97375) (end 154.60875 46.51375) (width 0.2) (layer "F.Cu") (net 23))
 (segment (start 154.60875 79.53375) (end 154.60875 82.07375) (width 0.2) (layer "F.Cu") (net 23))
 (segment (start 154.60875 71.91375) (end 154.60875 74.45375) (width 0.2) (layer "F.Cu") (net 23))
 (segment (start 154.60875 31.27375) (end 154.60875 33.81375) (width 0.2) (layer "F.Cu") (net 23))
 (segment (start 154.60875 59.21375) (end 154.60875 61.75375) (width 0.2) (layer "F.Cu") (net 23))
 (segment (start 109.71 82.07375) (end 115.7425 88.10625) (width 0.2) (layer "B.Cu") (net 23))
 (segment (start 151.11625 88.10625) (end 154.60875 84.61375) (width 0.2) (layer "B.Cu") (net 23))
 (segment (start 115.7425 88.10625) (end 151.11625 88.10625) (width 0.2) (layer "B.Cu") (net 23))
 (segment (start 100.0125 76.35875) (end 105.8465 70.52475) (width 0.2) (layer "B.Cu") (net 16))
 (segment (start 105.8465 70.52475) (end 105.8465 68.15725) (width 0.2) (layer "B.Cu") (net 16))
 (segment (start 105.8465 68.15725) (end 109.71 64.29375) (width 0.2) (layer "B.Cu") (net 16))
 (segment (start 150.01875 59.21375) (end 150.01875 56.67375) (width 0.2) (layer "F.Cu") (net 24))
 (segment (start 150.01875 41.43375) (end 150.01875 38.89375) (width 0.2) (layer "F.Cu") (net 24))
 (segment (start 150.01875 76.99375) (end 150.01875 74.45375) (width 0.2) (layer "F.Cu") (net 24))
 (segment (start 150.01875 43.97375) (end 150.01875 41.43375) (width 0.2) (layer "F.Cu") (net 24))
 (segment (start 150.01875 38.89375) (end 150.01875 36.35375) (width 0.2) (layer "F.Cu") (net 24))
 (segment (start 146.52625 88.10625) (end 150.01875 84.61375) (width 0.2) (layer "F.Cu") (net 24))
 (segment (start 150.01875 36.35375) (end 150.01875 33.81375) (width 0.2) (layer "F.Cu") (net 24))
 (segment (start 150.01875 33.81375) (end 150.01875 31.27375) (width 0.2) (layer "F.Cu") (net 24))
 (segment (start 150.01875 28.73375) (end 150.01875 26.19375) (width 0.2) (layer "F.Cu") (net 24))
 (segment (start 150.01875 69.37375) (end 150.01875 66.83375) (width 0.2) (layer "F.Cu") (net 24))
 (segment (start 150.01875 51.59375) (end 150.01875 49.05375) (width 0.2) (layer "F.Cu") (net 24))
 (segment (start 150.01875 64.29375) (end 150.01875 61.75375) (width 0.2) (layer "F.Cu") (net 24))
 (segment (start 150.01875 82.07375) (end 150.01875 79.53375) (width 0.2) (layer "F.Cu") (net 24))
 (segment (start 150.01875 71.91375) (end 150.01875 69.37375) (width 0.2) (layer "F.Cu") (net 24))
 (segment (start 150.01875 84.61375) (end 150.01875 82.07375) (width 0.2) (layer "F.Cu") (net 24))
 (segment (start 150.01875 64.29375) (end 150.01875 66.83375) (width 0.2) (layer "F.Cu") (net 24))
 (segment (start 150.01875 74.45375) (end 150.01875 71.91375) (width 0.2) (layer "F.Cu") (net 24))
 (segment (start 113.2025 88.10625) (end 146.52625 88.10625) (width 0.2) (layer "F.Cu") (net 24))
 (segment (start 150.01875 79.53375) (end 150.01875 76.99375) (width 0.2) (layer "F.Cu") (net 24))
 (segment (start 150.01875 61.75375) (end 150.01875 59.21375) (width 0.2) (layer "F.Cu") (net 24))
 (segment (start 109.71 84.61375) (end 113.2025 88.10625) (width 0.2) (layer "F.Cu") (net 24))
 (segment (start 150.01875 31.27375) (end 150.01875 28.73375) (width 0.2) (layer "F.Cu") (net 24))
 (segment (start 150.01875 46.51375) (end 150.01875 43.97375) (width 0.2) (layer "F.Cu") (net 24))
 (segment (start 150.01875 56.67375) (end 150.01875 54.13375) (width 0.2) (layer "F.Cu") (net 24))
 (segment (start 150.01875 54.13375) (end 150.01875 51.59375) (width 0.2) (layer "F.Cu") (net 24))
 (segment (start 150.01875 49.05375) (end 150.01875 46.51375) (width 0.2) (layer "F.Cu") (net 24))
 (segment (start 100.0125 78.89875) (end 108.3865 70.52475) (width 0.2) (layer "B.Cu") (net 17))
 (segment (start 108.3865 70.52475) (end 108.3865 68.15725) (width 0.2) (layer "B.Cu") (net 17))
 (segment (start 108.3865 68.15725) (end 109.71 66.83375) (width 0.2) (layer "B.Cu") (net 17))
 (segment (start 105.265 83.97875) (end 109.71 79.53375) (width 0.2) (layer "B.Cu") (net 22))
 (segment (start 100.0125 83.97875) (end 105.265 83.97875) (width 0.2) (layer "B.Cu") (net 22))
 (segment (start 131.14125 43.97375) (end 145.42875 43.97375) (width 0.2) (layer "F.Cu") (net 32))
 (segment (start 131.14125 38.89375) (end 145.42875 38.89375) (width 0.2) (layer "F.Cu") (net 30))
 (segment (start 145.42875 82.07375) (end 131.14125 82.07375) (width 0.2) (layer "F.Cu") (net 47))
 (segment (start 131.14125 69.37375) (end 145.42875 69.37375) (width 0.2) (layer "F.Cu") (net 42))
 (segment (start 131.14125 79.53375) (end 145.42875 79.53375) (width 0.2) (layer "F.Cu") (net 46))
 (segment (start 131.14125 64.29375) (end 145.42875 64.29375) (width 0.2) (layer "F.Cu") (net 40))
 (segment (start 131.14125 71.91375) (end 145.42875 71.91375) (width 0.2) (layer "F.Cu") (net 43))
 (segment (start 145.42875 51.59375) (end 131.14125 51.59375) (width 0.2) (layer "F.Cu") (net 35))
 (segment (start 131.14125 36.35375) (end 145.42875 36.35375) (width 0.2) (layer "F.Cu") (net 29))
 (segment (start 131.14125 61.75375) (end 145.42875 61.75375) (width 0.2) (layer "F.Cu") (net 39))
 (segment (start 145.42875 56.67375) (end 131.14125 56.67375) (width 0.2) (layer "F.Cu") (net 37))
 (segment (start 131.14125 26.19375) (end 145.42875 26.19375) (width 0.2) (layer "F.Cu") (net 25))
 (segment (start 131.14125 59.21375) (end 145.42875 59.21375) (width 0.2) (layer "F.Cu") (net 38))
 (segment (start 131.14125 49.05375) (end 145.42875 49.05375) (width 0.2) (layer "F.Cu") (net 34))
 (segment (start 131.14125 31.27375) (end 145.42875 31.27375) (width 0.2) (layer "F.Cu") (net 27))
 (segment (start 145.42875 46.51375) (end 131.14125 46.51375) (width 0.2) (layer "F.Cu") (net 33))
 (segment (start 145.42875 84.61375) (end 131.14125 84.61375) (width 0.2) (layer "F.Cu") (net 48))
 (segment (start 145.42875 41.43375) (end 131.14125 41.43375) (width 0.2) (layer "F.Cu") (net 31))
 (segment (start 131.14125 66.83375) (end 145.42875 66.83375) (width 0.2) (layer "F.Cu") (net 41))
 (segment (start 131.14125 54.13375) (end 145.42875 54.13375) (width 0.2) (layer "F.Cu") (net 36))
 (segment (start 131.14125 76.99375) (end 145.42875 76.99375) (width 0.2) (layer "F.Cu") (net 45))
 (segment (start 145.42875 33.81375) (end 131.14125 33.81375) (width 0.2) (layer "F.Cu") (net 28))
 (segment (start 145.42875 28.73375) (end 131.14125 28.73375) (width 0.2) (layer "F.Cu") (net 26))
 (segment (start 131.14125 74.45375) (end 145.42875 74.45375) (width 0.2) (layer "F.Cu") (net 44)))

